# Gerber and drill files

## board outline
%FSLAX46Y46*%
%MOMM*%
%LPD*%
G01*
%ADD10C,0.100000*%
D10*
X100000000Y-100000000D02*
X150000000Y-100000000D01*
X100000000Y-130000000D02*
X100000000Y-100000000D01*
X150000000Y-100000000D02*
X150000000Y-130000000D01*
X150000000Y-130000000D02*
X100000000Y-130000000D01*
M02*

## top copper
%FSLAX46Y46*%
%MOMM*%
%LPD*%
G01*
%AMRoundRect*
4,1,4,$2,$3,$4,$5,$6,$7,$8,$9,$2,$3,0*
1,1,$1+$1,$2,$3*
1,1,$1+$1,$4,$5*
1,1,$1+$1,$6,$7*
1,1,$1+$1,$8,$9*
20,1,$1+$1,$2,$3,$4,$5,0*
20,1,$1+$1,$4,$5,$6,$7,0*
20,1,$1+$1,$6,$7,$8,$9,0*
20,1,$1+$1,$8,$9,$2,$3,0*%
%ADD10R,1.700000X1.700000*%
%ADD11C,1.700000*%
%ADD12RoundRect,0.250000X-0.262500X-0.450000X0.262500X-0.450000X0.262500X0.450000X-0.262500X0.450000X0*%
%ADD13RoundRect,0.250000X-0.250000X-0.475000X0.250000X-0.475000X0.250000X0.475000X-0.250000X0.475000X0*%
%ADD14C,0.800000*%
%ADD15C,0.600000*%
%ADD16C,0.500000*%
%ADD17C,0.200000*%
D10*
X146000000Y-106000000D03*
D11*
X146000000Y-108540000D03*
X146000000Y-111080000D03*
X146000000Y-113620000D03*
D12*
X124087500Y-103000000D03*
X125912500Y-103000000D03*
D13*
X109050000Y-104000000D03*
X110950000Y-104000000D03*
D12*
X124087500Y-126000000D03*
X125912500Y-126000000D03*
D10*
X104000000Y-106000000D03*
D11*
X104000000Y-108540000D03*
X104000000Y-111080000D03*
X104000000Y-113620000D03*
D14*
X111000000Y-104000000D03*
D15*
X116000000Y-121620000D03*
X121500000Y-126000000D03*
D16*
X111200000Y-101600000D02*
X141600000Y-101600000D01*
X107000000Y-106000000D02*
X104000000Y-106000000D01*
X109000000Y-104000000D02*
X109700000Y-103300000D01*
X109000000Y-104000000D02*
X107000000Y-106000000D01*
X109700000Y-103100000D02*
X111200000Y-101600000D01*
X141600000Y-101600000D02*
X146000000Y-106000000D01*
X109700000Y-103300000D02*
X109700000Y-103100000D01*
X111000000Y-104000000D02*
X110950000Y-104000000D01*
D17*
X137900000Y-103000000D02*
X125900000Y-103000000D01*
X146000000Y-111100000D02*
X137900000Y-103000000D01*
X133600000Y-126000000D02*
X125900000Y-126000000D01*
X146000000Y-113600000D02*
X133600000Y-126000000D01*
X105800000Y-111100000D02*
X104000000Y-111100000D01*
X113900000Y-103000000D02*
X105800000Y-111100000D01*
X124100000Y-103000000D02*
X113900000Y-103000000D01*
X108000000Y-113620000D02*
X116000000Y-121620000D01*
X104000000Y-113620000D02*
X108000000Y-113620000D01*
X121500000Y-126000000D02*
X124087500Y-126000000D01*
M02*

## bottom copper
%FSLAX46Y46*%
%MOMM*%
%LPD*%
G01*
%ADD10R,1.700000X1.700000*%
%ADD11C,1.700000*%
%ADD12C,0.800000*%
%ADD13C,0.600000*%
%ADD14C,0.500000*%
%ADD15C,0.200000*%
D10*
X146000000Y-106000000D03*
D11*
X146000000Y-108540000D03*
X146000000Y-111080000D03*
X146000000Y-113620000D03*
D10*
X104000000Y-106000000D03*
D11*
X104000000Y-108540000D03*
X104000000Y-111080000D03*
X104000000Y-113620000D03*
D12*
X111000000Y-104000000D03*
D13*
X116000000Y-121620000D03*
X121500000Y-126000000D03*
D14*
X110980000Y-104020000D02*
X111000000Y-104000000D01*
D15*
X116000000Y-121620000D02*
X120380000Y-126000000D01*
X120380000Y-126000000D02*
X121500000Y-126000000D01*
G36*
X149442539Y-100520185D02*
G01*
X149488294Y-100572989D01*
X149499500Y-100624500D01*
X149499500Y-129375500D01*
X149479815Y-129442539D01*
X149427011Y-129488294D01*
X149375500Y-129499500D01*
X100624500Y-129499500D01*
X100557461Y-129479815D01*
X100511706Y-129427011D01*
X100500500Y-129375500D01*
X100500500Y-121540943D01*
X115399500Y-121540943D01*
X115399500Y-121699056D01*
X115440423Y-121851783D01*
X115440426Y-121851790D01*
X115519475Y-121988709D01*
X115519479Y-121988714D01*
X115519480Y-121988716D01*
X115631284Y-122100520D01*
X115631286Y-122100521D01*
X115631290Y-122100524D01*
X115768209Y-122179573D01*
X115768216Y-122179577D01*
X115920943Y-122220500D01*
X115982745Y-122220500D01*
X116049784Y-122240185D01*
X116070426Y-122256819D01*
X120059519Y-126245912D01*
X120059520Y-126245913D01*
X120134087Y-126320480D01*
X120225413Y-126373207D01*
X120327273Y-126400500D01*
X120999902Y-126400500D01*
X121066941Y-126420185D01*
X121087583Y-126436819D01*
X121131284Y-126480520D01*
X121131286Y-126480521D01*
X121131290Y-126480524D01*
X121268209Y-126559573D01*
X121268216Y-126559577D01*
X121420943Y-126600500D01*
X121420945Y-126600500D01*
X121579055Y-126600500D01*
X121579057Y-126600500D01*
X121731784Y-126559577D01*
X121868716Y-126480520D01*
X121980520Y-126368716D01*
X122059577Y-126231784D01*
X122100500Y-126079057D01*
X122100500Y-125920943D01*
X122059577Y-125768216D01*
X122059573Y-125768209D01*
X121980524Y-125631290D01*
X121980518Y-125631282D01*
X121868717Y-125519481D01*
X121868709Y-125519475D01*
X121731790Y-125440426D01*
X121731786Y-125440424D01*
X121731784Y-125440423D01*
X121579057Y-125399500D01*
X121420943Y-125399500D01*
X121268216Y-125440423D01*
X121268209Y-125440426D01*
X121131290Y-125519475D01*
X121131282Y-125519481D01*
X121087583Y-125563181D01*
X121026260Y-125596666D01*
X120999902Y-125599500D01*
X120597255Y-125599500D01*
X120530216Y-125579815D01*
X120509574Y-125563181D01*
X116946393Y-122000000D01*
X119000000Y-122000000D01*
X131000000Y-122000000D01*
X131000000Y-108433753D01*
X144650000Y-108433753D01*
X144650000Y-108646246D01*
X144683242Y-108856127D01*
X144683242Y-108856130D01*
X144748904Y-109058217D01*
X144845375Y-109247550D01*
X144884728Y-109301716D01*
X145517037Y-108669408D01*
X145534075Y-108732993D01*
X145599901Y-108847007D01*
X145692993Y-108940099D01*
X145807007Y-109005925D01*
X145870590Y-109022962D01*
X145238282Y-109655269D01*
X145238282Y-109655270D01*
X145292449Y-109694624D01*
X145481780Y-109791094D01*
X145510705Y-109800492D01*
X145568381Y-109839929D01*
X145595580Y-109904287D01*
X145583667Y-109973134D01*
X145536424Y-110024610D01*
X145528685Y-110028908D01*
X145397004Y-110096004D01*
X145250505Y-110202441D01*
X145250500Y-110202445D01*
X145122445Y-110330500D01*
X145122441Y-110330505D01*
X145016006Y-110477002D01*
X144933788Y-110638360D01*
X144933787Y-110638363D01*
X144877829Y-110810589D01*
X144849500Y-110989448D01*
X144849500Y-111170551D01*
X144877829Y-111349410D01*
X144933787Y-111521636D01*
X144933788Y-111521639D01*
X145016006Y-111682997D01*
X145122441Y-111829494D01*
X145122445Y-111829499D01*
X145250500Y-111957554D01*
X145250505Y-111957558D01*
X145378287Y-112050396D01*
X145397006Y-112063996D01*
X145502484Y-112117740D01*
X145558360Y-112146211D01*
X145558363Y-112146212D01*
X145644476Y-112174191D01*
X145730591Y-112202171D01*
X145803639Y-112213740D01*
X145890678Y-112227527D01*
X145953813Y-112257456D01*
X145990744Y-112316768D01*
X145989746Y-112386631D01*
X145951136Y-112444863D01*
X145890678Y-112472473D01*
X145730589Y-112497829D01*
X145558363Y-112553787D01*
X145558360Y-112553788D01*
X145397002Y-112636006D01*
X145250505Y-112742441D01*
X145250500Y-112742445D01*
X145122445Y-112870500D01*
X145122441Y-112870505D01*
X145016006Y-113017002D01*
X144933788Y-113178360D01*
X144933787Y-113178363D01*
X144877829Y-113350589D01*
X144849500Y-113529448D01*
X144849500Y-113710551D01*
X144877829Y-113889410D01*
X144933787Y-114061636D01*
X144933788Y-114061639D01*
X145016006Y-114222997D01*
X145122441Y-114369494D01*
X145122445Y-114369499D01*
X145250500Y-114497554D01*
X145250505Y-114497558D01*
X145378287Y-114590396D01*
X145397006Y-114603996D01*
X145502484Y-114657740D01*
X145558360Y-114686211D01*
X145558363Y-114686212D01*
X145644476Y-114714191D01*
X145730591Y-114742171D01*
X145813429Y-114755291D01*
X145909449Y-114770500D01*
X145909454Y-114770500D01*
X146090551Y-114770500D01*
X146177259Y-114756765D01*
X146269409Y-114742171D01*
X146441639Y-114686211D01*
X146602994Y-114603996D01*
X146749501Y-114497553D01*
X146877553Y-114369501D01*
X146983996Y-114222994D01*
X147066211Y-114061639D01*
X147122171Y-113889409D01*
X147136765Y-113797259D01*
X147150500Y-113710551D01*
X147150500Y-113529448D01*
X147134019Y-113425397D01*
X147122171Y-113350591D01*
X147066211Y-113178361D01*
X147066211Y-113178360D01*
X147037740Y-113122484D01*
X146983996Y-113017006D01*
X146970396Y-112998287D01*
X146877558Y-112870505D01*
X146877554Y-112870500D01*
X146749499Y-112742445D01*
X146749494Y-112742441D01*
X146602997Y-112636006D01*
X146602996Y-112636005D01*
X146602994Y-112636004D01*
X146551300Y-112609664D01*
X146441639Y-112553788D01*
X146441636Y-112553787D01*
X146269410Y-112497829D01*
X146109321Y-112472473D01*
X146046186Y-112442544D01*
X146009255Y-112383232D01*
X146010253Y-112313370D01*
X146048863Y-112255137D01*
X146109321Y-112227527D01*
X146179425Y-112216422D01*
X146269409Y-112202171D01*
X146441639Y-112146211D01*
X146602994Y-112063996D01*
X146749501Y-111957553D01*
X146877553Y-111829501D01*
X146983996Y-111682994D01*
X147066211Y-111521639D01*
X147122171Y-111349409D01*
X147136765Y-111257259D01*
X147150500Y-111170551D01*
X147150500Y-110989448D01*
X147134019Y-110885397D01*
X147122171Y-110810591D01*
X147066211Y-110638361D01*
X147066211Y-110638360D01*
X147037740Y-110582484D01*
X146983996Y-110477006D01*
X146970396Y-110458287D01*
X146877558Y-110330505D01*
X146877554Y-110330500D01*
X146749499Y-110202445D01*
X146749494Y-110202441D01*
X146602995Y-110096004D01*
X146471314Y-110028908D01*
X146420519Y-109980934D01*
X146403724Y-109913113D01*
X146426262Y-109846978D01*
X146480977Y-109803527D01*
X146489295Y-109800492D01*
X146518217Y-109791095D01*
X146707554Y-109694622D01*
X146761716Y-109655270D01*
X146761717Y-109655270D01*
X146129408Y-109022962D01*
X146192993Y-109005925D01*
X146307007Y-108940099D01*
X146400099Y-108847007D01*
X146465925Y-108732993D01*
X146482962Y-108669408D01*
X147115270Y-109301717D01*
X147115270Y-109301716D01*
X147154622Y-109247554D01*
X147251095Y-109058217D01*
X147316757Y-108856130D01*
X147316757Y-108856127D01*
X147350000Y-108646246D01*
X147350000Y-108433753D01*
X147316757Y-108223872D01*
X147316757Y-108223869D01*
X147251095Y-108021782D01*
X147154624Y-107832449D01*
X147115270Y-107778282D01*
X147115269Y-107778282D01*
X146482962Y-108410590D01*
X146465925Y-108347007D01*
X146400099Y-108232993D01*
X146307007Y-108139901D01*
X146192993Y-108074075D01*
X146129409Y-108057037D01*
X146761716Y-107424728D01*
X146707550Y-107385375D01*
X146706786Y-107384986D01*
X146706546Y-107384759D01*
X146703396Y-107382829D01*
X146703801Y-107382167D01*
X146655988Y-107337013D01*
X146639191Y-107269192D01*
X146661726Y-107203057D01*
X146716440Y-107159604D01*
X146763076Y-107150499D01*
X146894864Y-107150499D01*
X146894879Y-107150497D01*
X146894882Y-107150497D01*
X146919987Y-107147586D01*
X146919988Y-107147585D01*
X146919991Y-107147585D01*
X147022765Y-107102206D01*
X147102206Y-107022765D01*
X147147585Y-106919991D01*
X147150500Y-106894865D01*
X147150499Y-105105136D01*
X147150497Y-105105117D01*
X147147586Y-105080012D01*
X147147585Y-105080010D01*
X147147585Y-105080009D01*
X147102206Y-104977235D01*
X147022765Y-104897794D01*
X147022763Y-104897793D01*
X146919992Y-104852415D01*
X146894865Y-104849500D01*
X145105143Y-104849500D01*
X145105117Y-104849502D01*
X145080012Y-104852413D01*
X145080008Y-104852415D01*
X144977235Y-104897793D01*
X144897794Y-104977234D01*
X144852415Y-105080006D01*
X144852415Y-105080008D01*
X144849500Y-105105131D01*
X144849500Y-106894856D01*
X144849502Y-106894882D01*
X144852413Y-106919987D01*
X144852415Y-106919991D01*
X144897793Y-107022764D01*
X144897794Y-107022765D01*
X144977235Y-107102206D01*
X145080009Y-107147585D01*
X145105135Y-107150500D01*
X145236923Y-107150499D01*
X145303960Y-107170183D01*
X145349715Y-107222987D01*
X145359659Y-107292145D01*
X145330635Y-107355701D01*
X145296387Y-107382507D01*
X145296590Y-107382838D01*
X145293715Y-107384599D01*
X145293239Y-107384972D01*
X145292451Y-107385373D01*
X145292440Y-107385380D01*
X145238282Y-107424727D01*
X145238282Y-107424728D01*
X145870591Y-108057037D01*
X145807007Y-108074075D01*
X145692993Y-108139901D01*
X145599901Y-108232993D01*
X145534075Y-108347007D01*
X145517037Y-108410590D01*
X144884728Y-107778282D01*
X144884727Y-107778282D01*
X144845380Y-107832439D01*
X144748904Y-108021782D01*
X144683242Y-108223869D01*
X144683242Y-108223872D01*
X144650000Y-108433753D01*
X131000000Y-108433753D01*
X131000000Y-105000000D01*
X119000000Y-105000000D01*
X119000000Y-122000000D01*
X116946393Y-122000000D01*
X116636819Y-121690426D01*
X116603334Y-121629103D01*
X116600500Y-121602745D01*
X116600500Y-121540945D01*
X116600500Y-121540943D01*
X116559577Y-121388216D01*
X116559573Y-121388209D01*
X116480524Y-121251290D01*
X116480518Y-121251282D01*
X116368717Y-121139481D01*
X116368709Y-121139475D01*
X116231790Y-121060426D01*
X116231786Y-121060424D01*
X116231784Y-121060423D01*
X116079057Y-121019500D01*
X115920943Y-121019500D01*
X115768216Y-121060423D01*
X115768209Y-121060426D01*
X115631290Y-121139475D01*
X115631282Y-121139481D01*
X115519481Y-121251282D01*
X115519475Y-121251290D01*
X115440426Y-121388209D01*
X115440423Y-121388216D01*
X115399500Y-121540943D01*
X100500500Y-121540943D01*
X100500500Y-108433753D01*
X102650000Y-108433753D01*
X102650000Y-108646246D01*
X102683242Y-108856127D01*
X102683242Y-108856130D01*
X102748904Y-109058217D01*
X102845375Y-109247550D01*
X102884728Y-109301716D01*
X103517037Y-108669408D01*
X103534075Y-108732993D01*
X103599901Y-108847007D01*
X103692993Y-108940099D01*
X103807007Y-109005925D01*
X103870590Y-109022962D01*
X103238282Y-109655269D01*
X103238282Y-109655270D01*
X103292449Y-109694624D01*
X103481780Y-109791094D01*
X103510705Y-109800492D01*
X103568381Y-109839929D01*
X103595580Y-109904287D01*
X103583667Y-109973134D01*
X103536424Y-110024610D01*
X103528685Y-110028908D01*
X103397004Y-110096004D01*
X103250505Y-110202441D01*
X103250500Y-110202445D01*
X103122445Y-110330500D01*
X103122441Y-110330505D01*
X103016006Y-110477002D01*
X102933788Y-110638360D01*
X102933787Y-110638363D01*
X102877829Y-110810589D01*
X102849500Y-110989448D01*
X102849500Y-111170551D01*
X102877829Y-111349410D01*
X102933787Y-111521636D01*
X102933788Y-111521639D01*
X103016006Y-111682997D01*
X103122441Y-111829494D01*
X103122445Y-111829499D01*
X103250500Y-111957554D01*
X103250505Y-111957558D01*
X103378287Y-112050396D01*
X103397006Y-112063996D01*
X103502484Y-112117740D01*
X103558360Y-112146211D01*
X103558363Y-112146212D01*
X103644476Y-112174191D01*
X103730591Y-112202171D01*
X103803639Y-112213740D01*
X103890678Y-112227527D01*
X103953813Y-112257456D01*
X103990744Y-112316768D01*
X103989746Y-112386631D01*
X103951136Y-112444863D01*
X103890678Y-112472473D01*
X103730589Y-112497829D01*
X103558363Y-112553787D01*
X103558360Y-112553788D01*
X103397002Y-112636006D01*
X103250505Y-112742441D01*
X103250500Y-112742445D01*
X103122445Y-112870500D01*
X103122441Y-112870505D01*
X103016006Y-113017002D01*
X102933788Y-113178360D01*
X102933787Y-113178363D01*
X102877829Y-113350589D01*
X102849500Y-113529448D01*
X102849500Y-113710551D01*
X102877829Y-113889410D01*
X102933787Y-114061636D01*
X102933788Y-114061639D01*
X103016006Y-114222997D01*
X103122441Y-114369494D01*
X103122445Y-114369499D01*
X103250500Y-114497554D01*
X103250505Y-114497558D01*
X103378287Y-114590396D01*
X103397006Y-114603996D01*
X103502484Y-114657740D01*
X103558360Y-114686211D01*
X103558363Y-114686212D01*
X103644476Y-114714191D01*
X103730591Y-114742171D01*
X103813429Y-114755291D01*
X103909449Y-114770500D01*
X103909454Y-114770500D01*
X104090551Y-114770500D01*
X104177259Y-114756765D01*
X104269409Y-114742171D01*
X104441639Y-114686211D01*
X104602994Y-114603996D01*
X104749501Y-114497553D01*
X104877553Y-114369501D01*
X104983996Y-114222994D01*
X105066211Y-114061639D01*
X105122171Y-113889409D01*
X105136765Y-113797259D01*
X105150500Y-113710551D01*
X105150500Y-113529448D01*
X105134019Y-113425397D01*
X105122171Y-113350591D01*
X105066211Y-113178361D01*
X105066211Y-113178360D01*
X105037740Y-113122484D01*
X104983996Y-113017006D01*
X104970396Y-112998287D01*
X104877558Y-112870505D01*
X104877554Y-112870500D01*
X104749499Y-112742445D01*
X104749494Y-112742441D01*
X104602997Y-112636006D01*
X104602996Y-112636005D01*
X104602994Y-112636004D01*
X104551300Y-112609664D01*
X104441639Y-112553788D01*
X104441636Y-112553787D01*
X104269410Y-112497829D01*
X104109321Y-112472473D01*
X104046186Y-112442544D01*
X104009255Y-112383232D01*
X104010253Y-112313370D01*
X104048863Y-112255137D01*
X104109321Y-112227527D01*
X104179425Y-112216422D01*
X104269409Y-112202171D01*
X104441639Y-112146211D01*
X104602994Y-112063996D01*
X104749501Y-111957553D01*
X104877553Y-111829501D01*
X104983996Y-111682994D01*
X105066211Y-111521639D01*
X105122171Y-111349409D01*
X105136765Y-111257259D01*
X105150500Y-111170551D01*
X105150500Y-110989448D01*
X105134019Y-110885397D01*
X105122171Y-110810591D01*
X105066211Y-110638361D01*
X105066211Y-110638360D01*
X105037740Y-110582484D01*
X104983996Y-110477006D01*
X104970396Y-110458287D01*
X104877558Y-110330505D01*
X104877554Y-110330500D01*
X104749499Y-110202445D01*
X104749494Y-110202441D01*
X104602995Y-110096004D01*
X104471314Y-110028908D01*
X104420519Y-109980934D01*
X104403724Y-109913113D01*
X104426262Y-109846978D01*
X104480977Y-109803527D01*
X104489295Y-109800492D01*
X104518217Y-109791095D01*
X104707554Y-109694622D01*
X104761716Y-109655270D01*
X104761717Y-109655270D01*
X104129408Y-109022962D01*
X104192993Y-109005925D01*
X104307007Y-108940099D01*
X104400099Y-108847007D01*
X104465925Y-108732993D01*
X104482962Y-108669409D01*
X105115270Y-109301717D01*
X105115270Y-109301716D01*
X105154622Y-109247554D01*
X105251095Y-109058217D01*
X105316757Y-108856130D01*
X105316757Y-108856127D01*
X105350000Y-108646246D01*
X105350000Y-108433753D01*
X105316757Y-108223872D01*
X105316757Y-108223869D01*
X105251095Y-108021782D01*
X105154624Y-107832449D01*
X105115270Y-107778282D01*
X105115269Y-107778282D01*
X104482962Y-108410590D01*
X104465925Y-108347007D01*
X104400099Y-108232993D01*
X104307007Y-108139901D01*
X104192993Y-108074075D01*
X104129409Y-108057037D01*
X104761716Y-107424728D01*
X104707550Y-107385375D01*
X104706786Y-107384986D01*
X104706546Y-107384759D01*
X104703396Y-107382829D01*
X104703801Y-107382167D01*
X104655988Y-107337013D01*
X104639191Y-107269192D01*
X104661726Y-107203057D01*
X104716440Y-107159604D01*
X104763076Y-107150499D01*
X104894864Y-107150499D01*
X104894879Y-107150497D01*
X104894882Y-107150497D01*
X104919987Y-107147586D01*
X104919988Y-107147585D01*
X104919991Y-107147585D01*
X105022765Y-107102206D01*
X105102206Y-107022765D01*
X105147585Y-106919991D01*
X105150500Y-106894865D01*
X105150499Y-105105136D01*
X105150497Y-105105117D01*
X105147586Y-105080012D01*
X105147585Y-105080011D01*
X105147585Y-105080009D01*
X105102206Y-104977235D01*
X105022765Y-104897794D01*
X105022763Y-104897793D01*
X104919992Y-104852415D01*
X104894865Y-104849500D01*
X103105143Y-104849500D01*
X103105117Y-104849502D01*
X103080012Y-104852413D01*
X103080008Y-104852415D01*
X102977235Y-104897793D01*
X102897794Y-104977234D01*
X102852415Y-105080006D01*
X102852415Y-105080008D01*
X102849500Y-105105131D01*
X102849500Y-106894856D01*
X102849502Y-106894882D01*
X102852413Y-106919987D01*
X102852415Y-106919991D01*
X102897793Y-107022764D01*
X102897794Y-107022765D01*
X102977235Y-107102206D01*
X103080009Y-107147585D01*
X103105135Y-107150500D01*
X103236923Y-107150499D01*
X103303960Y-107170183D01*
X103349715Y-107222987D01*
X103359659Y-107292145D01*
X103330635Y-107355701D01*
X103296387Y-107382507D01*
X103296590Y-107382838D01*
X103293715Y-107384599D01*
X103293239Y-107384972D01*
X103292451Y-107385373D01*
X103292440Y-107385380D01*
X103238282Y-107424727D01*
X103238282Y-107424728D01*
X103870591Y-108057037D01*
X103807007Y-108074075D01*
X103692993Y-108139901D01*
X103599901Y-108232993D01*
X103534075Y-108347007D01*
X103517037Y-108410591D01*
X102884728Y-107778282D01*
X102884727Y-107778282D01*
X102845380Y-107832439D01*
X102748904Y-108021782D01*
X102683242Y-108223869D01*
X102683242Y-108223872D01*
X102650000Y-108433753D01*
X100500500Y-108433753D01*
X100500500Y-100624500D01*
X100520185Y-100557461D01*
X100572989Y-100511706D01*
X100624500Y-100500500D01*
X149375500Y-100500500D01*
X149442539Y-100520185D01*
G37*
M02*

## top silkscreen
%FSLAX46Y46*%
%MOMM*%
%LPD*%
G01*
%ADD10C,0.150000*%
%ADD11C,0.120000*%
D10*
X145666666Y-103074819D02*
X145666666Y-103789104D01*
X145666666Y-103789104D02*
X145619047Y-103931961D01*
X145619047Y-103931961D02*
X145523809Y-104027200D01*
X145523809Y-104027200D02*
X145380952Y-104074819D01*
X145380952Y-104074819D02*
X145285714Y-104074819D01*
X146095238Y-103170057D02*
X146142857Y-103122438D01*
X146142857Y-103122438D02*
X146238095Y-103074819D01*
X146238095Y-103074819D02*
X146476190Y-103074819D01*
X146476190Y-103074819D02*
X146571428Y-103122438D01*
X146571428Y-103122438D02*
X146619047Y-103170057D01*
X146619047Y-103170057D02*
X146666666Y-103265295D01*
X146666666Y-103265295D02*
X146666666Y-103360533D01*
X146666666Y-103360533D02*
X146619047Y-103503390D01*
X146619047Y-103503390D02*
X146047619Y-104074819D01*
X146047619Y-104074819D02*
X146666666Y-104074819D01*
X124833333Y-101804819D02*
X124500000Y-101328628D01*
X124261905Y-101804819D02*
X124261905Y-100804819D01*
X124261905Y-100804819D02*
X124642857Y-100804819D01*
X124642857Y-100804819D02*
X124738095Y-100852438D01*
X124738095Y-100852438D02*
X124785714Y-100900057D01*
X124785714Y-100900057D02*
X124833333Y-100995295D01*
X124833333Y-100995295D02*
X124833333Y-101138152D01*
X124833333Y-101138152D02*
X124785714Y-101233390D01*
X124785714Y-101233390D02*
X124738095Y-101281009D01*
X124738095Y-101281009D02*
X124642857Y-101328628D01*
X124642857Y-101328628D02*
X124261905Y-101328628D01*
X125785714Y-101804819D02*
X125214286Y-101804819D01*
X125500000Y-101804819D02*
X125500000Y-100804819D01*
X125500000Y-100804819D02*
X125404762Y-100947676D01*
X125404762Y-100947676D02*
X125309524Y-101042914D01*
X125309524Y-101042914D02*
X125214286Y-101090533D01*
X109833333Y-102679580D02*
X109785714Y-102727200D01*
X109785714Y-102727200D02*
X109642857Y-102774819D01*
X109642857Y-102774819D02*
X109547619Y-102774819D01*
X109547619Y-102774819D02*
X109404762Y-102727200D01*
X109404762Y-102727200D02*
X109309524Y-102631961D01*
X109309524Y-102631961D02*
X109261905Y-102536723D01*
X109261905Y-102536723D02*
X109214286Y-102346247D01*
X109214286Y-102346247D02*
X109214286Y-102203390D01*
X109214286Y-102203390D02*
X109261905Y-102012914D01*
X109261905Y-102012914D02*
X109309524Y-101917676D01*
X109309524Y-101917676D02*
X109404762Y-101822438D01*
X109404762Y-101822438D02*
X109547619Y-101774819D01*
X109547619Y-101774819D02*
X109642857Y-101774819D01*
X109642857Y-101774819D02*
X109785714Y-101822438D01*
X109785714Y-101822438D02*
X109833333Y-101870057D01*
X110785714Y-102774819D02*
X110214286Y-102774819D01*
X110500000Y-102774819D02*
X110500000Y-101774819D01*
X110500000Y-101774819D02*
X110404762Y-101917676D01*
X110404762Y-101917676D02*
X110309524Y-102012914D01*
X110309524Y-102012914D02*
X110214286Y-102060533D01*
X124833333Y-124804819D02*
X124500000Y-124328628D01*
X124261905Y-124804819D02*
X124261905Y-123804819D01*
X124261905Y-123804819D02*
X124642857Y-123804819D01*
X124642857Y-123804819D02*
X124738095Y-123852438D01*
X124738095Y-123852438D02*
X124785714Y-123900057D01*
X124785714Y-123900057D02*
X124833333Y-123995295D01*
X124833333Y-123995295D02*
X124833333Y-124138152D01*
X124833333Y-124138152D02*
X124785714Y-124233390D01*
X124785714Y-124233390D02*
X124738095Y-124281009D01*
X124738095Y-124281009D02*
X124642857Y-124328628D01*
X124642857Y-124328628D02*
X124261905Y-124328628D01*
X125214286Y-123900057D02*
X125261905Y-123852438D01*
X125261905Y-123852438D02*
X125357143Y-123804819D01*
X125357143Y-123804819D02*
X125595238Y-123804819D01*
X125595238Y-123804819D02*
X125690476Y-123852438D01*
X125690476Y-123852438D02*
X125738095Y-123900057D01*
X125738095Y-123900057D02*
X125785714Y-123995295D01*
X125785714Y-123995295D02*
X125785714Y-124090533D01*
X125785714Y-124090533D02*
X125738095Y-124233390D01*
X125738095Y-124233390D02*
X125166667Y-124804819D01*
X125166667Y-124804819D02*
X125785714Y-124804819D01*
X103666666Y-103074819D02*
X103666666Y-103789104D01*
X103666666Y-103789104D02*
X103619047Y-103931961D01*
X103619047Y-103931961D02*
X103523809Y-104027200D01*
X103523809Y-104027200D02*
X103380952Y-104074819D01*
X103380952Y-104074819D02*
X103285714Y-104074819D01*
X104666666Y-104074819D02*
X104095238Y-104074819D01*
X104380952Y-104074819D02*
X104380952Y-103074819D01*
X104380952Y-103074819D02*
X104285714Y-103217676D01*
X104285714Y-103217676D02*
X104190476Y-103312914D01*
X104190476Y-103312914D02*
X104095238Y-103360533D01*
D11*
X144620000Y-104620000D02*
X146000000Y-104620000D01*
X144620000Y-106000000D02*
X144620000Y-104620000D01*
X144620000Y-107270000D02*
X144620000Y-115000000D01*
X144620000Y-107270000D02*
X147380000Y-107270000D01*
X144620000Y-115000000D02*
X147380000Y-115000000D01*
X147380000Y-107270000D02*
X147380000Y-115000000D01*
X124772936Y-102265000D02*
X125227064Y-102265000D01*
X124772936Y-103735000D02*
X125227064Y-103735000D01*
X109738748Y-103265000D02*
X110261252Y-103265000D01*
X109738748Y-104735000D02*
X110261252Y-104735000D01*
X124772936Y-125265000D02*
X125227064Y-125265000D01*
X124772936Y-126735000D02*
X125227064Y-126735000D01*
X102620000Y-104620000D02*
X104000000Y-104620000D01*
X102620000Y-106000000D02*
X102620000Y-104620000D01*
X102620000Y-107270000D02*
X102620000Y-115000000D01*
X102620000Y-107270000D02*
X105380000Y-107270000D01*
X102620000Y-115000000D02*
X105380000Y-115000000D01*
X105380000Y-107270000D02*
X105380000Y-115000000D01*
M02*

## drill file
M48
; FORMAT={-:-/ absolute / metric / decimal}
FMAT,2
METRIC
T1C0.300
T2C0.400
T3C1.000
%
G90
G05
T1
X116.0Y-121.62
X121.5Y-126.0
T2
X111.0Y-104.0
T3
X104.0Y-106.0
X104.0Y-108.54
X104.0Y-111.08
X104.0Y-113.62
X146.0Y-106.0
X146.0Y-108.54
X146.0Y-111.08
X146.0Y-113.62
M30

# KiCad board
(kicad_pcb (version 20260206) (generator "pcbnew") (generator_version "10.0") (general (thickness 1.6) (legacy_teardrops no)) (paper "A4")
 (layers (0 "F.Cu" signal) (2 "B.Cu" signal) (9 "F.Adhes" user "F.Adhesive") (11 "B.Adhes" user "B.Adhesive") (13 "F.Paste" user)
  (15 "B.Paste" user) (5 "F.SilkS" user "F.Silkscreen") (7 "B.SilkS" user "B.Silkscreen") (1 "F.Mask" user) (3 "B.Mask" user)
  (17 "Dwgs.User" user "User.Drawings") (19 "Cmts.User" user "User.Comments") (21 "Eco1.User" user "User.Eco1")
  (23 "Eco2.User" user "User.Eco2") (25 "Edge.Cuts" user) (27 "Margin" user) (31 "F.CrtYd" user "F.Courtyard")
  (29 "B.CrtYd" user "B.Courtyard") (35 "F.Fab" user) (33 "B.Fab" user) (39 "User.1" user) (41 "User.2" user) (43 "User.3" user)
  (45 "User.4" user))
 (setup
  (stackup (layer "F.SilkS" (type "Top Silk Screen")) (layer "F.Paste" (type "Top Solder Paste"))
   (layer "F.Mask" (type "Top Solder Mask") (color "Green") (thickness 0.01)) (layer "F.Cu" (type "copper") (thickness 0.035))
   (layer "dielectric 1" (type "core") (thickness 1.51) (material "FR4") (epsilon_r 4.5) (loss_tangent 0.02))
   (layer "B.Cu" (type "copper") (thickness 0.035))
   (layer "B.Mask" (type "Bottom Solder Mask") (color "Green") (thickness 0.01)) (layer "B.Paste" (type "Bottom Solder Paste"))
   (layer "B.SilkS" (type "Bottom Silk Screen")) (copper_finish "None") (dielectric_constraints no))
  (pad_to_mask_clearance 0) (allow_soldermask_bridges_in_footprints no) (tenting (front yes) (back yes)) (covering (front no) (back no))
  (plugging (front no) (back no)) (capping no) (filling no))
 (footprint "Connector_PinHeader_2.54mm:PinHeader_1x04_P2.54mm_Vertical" (layer "F.Cu") (at 146 106)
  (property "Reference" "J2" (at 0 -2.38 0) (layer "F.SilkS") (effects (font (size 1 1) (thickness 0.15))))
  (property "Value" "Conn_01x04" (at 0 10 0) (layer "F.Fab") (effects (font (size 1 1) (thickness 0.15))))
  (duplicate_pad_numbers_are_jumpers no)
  (fp_line (start -1.38 -1.38) (end 0 -1.38) (stroke (width 0.12) (type solid)) (layer "F.SilkS"))
  (fp_line (start -1.38 0) (end -1.38 -1.38) (stroke (width 0.12) (type solid)) (layer "F.SilkS"))
  (fp_line (start -1.38 1.27) (end -1.38 9) (stroke (width 0.12) (type solid)) (layer "F.SilkS"))
  (fp_line (start -1.38 1.27) (end 1.38 1.27) (stroke (width 0.12) (type solid)) (layer "F.SilkS"))
  (fp_line (start -1.38 9) (end 1.38 9) (stroke (width 0.12) (type solid)) (layer "F.SilkS"))
  (fp_line (start 1.38 1.27) (end 1.38 9) (stroke (width 0.12) (type solid)) (layer "F.SilkS"))
  (pad "1" thru_hole rect (at 0 0) (size 1.7 1.7) (drill 1) (layers "*.Cu" "*.Mask") (remove_unused_layers no) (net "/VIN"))
  (pad "2" thru_hole circle (at 0 2.54) (size 1.7 1.7) (drill 1) (layers "*.Cu" "*.Mask") (remove_unused_layers no) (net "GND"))
  (pad "3" thru_hole circle (at 0 5.08) (size 1.7 1.7) (drill 1) (layers "*.Cu" "*.Mask") (remove_unused_layers no) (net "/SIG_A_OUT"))
  (pad "4" thru_hole circle (at 0 7.62) (size 1.7 1.7) (drill 1) (layers "*.Cu" "*.Mask") (remove_unused_layers no) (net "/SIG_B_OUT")))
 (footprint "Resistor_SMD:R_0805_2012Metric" (layer "F.Cu") (at 125 103)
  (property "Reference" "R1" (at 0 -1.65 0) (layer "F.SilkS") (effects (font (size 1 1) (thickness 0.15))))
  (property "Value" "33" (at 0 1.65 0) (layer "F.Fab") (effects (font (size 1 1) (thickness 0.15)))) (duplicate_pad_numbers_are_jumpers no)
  (fp_line (start -0.227064 -0.735) (end 0.227064 -0.735) (stroke (width 0.12) (type solid)) (layer "F.SilkS"))
  (fp_line (start -0.227064 0.735) (end 0.227064 0.735) (stroke (width 0.12) (type solid)) (layer "F.SilkS"))
  (pad "1" smd roundrect (at -0.9125 0) (size 1.025 1.4) (layers "F.Cu" "F.Mask" "F.Paste") (roundrect_rratio 0.243902) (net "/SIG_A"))
  (pad "2" smd roundrect (at 0.9125 0) (size 1.025 1.4) (layers "F.Cu" "F.Mask" "F.Paste") (roundrect_rratio 0.243902) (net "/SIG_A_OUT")))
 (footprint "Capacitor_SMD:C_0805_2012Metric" (layer "F.Cu") (at 110 104)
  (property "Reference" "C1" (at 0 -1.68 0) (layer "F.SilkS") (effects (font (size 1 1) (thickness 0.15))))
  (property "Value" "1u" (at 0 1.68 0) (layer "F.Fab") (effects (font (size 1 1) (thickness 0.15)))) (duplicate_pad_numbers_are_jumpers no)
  (fp_line (start -0.261252 -0.735) (end 0.261252 -0.735) (stroke (width 0.12) (type solid)) (layer "F.SilkS"))
  (fp_line (start -0.261252 0.735) (end 0.261252 0.735) (stroke (width 0.12) (type solid)) (layer "F.SilkS"))
  (pad "1" smd roundrect (at -0.95 0) (size 1 1.45) (layers "F.Cu" "F.Mask" "F.Paste") (roundrect_rratio 0.25) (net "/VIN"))
  (pad "2" smd roundrect (at 0.95 0) (size 1 1.45) (layers "F.Cu" "F.Mask" "F.Paste") (roundrect_rratio 0.25) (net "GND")))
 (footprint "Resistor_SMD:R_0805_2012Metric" (layer "F.Cu") (at 125 126)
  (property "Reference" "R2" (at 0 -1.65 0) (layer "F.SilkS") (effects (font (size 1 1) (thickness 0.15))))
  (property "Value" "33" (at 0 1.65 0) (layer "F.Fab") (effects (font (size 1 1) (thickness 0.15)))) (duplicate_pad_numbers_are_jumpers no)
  (fp_line (start -0.227064 -0.735) (end 0.227064 -0.735) (stroke (width 0.12) (type solid)) (layer "F.SilkS"))
  (fp_line (start -0.227064 0.735) (end 0.227064 0.735) (stroke (width 0.12) (type solid)) (layer "F.SilkS"))
  (pad "1" smd roundrect (at -0.9125 0) (size 1.025 1.4) (layers "F.Cu" "F.Mask" "F.Paste") (roundrect_rratio 0.243902) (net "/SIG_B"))
  (pad "2" smd roundrect (at 0.9125 0) (size 1.025 1.4) (layers "F.Cu" "F.Mask" "F.Paste") (roundrect_rratio 0.243902) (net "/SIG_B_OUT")))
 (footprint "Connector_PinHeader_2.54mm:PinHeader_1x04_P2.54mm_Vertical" (layer "F.Cu") (at 104 106)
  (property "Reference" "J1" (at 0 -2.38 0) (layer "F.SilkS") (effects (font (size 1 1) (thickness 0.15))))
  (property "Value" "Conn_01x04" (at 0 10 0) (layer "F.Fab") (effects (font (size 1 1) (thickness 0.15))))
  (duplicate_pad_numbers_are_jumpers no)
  (fp_line (start -1.38 -1.38) (end 0 -1.38) (stroke (width 0.12) (type solid)) (layer "F.SilkS"))
  (fp_line (start -1.38 0) (end -1.38 -1.38) (stroke (width 0.12) (type solid)) (layer "F.SilkS"))
  (fp_line (start -1.38 1.27) (end -1.38 9) (stroke (width 0.12) (type solid)) (layer "F.SilkS"))
  (fp_line (start -1.38 1.27) (end 1.38 1.27) (stroke (width 0.12) (type solid)) (layer "F.SilkS"))
  (fp_line (start -1.38 9) (end 1.38 9) (stroke (width 0.12) (type solid)) (layer "F.SilkS"))
  (fp_line (start 1.38 1.27) (end 1.38 9) (stroke (width 0.12) (type solid)) (layer "F.SilkS"))
  (pad "1" thru_hole rect (at 0 0) (size 1.7 1.7) (drill 1) (layers "*.Cu" "*.Mask") (remove_unused_layers no) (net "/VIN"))
  (pad "2" thru_hole circle (at 0 2.54) (size 1.7 1.7) (drill 1) (layers "*.Cu" "*.Mask") (remove_unused_layers no) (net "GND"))
  (pad "3" thru_hole circle (at 0 5.08) (size 1.7 1.7) (drill 1) (layers "*.Cu" "*.Mask") (remove_unused_layers no) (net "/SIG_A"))
  (pad "4" thru_hole circle (at 0 7.62) (size 1.7 1.7) (drill 1) (layers "*.Cu" "*.Mask") (remove_unused_layers no) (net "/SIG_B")))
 (gr_line (start 100 100) (end 150 100) (stroke (width 0.1) (type default)) (layer "Edge.Cuts"))
 (gr_line (start 100 130) (end 100 100) (stroke (width 0.1) (type default)) (layer "Edge.Cuts"))
 (gr_line (start 150 100) (end 150 130) (stroke (width 0.1) (type default)) (layer "Edge.Cuts"))
 (gr_line (start 150 130) (end 100 130) (stroke (width 0.1) (type default)) (layer "Edge.Cuts"))
 (segment (start 111.2 101.6) (end 141.6 101.6) (width 0.5) (layer "F.Cu") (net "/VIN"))
 (segment (start 107 106) (end 104 106) (width 0.5) (layer "F.Cu") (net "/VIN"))
 (segment (start 109 104) (end 109.7 103.3) (width 0.5) (layer "F.Cu") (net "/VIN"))
 (segment (start 109 104) (end 107 106) (width 0.5) (layer "F.Cu") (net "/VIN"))
 (segment (start 109.7 103.1) (end 111.2 101.6) (width 0.5) (layer "F.Cu") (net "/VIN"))
 (segment (start 141.6 101.6) (end 146 106) (width 0.5) (layer "F.Cu") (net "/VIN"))
 (segment (start 109.7 103.3) (end 109.7 103.1) (width 0.5) (layer "F.Cu") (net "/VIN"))
 (segment (start 111 104) (end 110.95 104) (width 0.5) (layer "F.Cu") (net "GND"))
 (via (at 111 104) (size 0.8) (drill 0.4) (layers "F.Cu" "B.Cu") (capping yes) (filling yes) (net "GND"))
 (segment (start 110.98 104.02) (end 111 104) (width 0.5) (layer "B.Cu") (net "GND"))
 (segment (start 137.9 103) (end 125.9 103) (width 0.2) (layer "F.Cu") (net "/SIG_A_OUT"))
 (segment (start 146 111.1) (end 137.9 103) (width 0.2) (layer "F.Cu") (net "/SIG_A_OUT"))
 (segment (start 133.6 126) (end 125.9 126) (width 0.2) (layer "F.Cu") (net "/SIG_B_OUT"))
 (segment (start 146 113.6) (end 133.6 126) (width 0.2) (layer "F.Cu") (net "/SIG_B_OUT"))
 (segment (start 105.8 111.1) (end 104 111.1) (width 0.2) (layer "F.Cu") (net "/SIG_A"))
 (segment (start 113.9 103) (end 105.8 111.1) (width 0.2) (layer "F.Cu") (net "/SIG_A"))
 (segment (start 124.1 103) (end 113.9 103) (width 0.2) (layer "F.Cu") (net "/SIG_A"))
 (segment (start 108 113.62) (end 116 121.62) (width 0.2) (locked yes) (layer "F.Cu") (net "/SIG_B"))
 (segment (start 104 113.62) (end 108 113.62) (width 0.2) (locked yes) (layer "F.Cu") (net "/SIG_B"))
 (segment (start 121.5 126) (end 124.0875 126) (width 0.2) (locked yes) (layer "F.Cu") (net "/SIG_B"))
 (via (at 116 121.62) (size 0.6) (drill 0.3) (layers "F.Cu" "B.Cu") (locked yes) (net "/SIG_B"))
 (via (at 121.5 126) (size 0.6) (drill 0.3) (layers "F.Cu" "B.Cu") (locked yes) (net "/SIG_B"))
 (segment (start 116 121.62) (end 120.38 126) (width 0.2) (locked yes) (layer "B.Cu") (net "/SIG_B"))
 (segment (start 120.38 126) (end 121.5 126) (width 0.2) (locked yes) (layer "B.Cu") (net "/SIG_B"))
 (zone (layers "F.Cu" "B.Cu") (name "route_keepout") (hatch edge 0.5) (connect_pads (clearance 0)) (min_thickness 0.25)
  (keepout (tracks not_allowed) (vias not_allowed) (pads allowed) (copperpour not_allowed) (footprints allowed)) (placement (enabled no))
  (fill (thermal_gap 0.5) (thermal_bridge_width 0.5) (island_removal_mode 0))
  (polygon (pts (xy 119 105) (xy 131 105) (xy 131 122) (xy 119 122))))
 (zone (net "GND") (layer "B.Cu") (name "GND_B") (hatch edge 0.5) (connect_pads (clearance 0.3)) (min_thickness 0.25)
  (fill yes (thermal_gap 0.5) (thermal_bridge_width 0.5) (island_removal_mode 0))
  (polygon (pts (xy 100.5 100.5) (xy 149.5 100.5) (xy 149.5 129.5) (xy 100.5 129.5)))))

